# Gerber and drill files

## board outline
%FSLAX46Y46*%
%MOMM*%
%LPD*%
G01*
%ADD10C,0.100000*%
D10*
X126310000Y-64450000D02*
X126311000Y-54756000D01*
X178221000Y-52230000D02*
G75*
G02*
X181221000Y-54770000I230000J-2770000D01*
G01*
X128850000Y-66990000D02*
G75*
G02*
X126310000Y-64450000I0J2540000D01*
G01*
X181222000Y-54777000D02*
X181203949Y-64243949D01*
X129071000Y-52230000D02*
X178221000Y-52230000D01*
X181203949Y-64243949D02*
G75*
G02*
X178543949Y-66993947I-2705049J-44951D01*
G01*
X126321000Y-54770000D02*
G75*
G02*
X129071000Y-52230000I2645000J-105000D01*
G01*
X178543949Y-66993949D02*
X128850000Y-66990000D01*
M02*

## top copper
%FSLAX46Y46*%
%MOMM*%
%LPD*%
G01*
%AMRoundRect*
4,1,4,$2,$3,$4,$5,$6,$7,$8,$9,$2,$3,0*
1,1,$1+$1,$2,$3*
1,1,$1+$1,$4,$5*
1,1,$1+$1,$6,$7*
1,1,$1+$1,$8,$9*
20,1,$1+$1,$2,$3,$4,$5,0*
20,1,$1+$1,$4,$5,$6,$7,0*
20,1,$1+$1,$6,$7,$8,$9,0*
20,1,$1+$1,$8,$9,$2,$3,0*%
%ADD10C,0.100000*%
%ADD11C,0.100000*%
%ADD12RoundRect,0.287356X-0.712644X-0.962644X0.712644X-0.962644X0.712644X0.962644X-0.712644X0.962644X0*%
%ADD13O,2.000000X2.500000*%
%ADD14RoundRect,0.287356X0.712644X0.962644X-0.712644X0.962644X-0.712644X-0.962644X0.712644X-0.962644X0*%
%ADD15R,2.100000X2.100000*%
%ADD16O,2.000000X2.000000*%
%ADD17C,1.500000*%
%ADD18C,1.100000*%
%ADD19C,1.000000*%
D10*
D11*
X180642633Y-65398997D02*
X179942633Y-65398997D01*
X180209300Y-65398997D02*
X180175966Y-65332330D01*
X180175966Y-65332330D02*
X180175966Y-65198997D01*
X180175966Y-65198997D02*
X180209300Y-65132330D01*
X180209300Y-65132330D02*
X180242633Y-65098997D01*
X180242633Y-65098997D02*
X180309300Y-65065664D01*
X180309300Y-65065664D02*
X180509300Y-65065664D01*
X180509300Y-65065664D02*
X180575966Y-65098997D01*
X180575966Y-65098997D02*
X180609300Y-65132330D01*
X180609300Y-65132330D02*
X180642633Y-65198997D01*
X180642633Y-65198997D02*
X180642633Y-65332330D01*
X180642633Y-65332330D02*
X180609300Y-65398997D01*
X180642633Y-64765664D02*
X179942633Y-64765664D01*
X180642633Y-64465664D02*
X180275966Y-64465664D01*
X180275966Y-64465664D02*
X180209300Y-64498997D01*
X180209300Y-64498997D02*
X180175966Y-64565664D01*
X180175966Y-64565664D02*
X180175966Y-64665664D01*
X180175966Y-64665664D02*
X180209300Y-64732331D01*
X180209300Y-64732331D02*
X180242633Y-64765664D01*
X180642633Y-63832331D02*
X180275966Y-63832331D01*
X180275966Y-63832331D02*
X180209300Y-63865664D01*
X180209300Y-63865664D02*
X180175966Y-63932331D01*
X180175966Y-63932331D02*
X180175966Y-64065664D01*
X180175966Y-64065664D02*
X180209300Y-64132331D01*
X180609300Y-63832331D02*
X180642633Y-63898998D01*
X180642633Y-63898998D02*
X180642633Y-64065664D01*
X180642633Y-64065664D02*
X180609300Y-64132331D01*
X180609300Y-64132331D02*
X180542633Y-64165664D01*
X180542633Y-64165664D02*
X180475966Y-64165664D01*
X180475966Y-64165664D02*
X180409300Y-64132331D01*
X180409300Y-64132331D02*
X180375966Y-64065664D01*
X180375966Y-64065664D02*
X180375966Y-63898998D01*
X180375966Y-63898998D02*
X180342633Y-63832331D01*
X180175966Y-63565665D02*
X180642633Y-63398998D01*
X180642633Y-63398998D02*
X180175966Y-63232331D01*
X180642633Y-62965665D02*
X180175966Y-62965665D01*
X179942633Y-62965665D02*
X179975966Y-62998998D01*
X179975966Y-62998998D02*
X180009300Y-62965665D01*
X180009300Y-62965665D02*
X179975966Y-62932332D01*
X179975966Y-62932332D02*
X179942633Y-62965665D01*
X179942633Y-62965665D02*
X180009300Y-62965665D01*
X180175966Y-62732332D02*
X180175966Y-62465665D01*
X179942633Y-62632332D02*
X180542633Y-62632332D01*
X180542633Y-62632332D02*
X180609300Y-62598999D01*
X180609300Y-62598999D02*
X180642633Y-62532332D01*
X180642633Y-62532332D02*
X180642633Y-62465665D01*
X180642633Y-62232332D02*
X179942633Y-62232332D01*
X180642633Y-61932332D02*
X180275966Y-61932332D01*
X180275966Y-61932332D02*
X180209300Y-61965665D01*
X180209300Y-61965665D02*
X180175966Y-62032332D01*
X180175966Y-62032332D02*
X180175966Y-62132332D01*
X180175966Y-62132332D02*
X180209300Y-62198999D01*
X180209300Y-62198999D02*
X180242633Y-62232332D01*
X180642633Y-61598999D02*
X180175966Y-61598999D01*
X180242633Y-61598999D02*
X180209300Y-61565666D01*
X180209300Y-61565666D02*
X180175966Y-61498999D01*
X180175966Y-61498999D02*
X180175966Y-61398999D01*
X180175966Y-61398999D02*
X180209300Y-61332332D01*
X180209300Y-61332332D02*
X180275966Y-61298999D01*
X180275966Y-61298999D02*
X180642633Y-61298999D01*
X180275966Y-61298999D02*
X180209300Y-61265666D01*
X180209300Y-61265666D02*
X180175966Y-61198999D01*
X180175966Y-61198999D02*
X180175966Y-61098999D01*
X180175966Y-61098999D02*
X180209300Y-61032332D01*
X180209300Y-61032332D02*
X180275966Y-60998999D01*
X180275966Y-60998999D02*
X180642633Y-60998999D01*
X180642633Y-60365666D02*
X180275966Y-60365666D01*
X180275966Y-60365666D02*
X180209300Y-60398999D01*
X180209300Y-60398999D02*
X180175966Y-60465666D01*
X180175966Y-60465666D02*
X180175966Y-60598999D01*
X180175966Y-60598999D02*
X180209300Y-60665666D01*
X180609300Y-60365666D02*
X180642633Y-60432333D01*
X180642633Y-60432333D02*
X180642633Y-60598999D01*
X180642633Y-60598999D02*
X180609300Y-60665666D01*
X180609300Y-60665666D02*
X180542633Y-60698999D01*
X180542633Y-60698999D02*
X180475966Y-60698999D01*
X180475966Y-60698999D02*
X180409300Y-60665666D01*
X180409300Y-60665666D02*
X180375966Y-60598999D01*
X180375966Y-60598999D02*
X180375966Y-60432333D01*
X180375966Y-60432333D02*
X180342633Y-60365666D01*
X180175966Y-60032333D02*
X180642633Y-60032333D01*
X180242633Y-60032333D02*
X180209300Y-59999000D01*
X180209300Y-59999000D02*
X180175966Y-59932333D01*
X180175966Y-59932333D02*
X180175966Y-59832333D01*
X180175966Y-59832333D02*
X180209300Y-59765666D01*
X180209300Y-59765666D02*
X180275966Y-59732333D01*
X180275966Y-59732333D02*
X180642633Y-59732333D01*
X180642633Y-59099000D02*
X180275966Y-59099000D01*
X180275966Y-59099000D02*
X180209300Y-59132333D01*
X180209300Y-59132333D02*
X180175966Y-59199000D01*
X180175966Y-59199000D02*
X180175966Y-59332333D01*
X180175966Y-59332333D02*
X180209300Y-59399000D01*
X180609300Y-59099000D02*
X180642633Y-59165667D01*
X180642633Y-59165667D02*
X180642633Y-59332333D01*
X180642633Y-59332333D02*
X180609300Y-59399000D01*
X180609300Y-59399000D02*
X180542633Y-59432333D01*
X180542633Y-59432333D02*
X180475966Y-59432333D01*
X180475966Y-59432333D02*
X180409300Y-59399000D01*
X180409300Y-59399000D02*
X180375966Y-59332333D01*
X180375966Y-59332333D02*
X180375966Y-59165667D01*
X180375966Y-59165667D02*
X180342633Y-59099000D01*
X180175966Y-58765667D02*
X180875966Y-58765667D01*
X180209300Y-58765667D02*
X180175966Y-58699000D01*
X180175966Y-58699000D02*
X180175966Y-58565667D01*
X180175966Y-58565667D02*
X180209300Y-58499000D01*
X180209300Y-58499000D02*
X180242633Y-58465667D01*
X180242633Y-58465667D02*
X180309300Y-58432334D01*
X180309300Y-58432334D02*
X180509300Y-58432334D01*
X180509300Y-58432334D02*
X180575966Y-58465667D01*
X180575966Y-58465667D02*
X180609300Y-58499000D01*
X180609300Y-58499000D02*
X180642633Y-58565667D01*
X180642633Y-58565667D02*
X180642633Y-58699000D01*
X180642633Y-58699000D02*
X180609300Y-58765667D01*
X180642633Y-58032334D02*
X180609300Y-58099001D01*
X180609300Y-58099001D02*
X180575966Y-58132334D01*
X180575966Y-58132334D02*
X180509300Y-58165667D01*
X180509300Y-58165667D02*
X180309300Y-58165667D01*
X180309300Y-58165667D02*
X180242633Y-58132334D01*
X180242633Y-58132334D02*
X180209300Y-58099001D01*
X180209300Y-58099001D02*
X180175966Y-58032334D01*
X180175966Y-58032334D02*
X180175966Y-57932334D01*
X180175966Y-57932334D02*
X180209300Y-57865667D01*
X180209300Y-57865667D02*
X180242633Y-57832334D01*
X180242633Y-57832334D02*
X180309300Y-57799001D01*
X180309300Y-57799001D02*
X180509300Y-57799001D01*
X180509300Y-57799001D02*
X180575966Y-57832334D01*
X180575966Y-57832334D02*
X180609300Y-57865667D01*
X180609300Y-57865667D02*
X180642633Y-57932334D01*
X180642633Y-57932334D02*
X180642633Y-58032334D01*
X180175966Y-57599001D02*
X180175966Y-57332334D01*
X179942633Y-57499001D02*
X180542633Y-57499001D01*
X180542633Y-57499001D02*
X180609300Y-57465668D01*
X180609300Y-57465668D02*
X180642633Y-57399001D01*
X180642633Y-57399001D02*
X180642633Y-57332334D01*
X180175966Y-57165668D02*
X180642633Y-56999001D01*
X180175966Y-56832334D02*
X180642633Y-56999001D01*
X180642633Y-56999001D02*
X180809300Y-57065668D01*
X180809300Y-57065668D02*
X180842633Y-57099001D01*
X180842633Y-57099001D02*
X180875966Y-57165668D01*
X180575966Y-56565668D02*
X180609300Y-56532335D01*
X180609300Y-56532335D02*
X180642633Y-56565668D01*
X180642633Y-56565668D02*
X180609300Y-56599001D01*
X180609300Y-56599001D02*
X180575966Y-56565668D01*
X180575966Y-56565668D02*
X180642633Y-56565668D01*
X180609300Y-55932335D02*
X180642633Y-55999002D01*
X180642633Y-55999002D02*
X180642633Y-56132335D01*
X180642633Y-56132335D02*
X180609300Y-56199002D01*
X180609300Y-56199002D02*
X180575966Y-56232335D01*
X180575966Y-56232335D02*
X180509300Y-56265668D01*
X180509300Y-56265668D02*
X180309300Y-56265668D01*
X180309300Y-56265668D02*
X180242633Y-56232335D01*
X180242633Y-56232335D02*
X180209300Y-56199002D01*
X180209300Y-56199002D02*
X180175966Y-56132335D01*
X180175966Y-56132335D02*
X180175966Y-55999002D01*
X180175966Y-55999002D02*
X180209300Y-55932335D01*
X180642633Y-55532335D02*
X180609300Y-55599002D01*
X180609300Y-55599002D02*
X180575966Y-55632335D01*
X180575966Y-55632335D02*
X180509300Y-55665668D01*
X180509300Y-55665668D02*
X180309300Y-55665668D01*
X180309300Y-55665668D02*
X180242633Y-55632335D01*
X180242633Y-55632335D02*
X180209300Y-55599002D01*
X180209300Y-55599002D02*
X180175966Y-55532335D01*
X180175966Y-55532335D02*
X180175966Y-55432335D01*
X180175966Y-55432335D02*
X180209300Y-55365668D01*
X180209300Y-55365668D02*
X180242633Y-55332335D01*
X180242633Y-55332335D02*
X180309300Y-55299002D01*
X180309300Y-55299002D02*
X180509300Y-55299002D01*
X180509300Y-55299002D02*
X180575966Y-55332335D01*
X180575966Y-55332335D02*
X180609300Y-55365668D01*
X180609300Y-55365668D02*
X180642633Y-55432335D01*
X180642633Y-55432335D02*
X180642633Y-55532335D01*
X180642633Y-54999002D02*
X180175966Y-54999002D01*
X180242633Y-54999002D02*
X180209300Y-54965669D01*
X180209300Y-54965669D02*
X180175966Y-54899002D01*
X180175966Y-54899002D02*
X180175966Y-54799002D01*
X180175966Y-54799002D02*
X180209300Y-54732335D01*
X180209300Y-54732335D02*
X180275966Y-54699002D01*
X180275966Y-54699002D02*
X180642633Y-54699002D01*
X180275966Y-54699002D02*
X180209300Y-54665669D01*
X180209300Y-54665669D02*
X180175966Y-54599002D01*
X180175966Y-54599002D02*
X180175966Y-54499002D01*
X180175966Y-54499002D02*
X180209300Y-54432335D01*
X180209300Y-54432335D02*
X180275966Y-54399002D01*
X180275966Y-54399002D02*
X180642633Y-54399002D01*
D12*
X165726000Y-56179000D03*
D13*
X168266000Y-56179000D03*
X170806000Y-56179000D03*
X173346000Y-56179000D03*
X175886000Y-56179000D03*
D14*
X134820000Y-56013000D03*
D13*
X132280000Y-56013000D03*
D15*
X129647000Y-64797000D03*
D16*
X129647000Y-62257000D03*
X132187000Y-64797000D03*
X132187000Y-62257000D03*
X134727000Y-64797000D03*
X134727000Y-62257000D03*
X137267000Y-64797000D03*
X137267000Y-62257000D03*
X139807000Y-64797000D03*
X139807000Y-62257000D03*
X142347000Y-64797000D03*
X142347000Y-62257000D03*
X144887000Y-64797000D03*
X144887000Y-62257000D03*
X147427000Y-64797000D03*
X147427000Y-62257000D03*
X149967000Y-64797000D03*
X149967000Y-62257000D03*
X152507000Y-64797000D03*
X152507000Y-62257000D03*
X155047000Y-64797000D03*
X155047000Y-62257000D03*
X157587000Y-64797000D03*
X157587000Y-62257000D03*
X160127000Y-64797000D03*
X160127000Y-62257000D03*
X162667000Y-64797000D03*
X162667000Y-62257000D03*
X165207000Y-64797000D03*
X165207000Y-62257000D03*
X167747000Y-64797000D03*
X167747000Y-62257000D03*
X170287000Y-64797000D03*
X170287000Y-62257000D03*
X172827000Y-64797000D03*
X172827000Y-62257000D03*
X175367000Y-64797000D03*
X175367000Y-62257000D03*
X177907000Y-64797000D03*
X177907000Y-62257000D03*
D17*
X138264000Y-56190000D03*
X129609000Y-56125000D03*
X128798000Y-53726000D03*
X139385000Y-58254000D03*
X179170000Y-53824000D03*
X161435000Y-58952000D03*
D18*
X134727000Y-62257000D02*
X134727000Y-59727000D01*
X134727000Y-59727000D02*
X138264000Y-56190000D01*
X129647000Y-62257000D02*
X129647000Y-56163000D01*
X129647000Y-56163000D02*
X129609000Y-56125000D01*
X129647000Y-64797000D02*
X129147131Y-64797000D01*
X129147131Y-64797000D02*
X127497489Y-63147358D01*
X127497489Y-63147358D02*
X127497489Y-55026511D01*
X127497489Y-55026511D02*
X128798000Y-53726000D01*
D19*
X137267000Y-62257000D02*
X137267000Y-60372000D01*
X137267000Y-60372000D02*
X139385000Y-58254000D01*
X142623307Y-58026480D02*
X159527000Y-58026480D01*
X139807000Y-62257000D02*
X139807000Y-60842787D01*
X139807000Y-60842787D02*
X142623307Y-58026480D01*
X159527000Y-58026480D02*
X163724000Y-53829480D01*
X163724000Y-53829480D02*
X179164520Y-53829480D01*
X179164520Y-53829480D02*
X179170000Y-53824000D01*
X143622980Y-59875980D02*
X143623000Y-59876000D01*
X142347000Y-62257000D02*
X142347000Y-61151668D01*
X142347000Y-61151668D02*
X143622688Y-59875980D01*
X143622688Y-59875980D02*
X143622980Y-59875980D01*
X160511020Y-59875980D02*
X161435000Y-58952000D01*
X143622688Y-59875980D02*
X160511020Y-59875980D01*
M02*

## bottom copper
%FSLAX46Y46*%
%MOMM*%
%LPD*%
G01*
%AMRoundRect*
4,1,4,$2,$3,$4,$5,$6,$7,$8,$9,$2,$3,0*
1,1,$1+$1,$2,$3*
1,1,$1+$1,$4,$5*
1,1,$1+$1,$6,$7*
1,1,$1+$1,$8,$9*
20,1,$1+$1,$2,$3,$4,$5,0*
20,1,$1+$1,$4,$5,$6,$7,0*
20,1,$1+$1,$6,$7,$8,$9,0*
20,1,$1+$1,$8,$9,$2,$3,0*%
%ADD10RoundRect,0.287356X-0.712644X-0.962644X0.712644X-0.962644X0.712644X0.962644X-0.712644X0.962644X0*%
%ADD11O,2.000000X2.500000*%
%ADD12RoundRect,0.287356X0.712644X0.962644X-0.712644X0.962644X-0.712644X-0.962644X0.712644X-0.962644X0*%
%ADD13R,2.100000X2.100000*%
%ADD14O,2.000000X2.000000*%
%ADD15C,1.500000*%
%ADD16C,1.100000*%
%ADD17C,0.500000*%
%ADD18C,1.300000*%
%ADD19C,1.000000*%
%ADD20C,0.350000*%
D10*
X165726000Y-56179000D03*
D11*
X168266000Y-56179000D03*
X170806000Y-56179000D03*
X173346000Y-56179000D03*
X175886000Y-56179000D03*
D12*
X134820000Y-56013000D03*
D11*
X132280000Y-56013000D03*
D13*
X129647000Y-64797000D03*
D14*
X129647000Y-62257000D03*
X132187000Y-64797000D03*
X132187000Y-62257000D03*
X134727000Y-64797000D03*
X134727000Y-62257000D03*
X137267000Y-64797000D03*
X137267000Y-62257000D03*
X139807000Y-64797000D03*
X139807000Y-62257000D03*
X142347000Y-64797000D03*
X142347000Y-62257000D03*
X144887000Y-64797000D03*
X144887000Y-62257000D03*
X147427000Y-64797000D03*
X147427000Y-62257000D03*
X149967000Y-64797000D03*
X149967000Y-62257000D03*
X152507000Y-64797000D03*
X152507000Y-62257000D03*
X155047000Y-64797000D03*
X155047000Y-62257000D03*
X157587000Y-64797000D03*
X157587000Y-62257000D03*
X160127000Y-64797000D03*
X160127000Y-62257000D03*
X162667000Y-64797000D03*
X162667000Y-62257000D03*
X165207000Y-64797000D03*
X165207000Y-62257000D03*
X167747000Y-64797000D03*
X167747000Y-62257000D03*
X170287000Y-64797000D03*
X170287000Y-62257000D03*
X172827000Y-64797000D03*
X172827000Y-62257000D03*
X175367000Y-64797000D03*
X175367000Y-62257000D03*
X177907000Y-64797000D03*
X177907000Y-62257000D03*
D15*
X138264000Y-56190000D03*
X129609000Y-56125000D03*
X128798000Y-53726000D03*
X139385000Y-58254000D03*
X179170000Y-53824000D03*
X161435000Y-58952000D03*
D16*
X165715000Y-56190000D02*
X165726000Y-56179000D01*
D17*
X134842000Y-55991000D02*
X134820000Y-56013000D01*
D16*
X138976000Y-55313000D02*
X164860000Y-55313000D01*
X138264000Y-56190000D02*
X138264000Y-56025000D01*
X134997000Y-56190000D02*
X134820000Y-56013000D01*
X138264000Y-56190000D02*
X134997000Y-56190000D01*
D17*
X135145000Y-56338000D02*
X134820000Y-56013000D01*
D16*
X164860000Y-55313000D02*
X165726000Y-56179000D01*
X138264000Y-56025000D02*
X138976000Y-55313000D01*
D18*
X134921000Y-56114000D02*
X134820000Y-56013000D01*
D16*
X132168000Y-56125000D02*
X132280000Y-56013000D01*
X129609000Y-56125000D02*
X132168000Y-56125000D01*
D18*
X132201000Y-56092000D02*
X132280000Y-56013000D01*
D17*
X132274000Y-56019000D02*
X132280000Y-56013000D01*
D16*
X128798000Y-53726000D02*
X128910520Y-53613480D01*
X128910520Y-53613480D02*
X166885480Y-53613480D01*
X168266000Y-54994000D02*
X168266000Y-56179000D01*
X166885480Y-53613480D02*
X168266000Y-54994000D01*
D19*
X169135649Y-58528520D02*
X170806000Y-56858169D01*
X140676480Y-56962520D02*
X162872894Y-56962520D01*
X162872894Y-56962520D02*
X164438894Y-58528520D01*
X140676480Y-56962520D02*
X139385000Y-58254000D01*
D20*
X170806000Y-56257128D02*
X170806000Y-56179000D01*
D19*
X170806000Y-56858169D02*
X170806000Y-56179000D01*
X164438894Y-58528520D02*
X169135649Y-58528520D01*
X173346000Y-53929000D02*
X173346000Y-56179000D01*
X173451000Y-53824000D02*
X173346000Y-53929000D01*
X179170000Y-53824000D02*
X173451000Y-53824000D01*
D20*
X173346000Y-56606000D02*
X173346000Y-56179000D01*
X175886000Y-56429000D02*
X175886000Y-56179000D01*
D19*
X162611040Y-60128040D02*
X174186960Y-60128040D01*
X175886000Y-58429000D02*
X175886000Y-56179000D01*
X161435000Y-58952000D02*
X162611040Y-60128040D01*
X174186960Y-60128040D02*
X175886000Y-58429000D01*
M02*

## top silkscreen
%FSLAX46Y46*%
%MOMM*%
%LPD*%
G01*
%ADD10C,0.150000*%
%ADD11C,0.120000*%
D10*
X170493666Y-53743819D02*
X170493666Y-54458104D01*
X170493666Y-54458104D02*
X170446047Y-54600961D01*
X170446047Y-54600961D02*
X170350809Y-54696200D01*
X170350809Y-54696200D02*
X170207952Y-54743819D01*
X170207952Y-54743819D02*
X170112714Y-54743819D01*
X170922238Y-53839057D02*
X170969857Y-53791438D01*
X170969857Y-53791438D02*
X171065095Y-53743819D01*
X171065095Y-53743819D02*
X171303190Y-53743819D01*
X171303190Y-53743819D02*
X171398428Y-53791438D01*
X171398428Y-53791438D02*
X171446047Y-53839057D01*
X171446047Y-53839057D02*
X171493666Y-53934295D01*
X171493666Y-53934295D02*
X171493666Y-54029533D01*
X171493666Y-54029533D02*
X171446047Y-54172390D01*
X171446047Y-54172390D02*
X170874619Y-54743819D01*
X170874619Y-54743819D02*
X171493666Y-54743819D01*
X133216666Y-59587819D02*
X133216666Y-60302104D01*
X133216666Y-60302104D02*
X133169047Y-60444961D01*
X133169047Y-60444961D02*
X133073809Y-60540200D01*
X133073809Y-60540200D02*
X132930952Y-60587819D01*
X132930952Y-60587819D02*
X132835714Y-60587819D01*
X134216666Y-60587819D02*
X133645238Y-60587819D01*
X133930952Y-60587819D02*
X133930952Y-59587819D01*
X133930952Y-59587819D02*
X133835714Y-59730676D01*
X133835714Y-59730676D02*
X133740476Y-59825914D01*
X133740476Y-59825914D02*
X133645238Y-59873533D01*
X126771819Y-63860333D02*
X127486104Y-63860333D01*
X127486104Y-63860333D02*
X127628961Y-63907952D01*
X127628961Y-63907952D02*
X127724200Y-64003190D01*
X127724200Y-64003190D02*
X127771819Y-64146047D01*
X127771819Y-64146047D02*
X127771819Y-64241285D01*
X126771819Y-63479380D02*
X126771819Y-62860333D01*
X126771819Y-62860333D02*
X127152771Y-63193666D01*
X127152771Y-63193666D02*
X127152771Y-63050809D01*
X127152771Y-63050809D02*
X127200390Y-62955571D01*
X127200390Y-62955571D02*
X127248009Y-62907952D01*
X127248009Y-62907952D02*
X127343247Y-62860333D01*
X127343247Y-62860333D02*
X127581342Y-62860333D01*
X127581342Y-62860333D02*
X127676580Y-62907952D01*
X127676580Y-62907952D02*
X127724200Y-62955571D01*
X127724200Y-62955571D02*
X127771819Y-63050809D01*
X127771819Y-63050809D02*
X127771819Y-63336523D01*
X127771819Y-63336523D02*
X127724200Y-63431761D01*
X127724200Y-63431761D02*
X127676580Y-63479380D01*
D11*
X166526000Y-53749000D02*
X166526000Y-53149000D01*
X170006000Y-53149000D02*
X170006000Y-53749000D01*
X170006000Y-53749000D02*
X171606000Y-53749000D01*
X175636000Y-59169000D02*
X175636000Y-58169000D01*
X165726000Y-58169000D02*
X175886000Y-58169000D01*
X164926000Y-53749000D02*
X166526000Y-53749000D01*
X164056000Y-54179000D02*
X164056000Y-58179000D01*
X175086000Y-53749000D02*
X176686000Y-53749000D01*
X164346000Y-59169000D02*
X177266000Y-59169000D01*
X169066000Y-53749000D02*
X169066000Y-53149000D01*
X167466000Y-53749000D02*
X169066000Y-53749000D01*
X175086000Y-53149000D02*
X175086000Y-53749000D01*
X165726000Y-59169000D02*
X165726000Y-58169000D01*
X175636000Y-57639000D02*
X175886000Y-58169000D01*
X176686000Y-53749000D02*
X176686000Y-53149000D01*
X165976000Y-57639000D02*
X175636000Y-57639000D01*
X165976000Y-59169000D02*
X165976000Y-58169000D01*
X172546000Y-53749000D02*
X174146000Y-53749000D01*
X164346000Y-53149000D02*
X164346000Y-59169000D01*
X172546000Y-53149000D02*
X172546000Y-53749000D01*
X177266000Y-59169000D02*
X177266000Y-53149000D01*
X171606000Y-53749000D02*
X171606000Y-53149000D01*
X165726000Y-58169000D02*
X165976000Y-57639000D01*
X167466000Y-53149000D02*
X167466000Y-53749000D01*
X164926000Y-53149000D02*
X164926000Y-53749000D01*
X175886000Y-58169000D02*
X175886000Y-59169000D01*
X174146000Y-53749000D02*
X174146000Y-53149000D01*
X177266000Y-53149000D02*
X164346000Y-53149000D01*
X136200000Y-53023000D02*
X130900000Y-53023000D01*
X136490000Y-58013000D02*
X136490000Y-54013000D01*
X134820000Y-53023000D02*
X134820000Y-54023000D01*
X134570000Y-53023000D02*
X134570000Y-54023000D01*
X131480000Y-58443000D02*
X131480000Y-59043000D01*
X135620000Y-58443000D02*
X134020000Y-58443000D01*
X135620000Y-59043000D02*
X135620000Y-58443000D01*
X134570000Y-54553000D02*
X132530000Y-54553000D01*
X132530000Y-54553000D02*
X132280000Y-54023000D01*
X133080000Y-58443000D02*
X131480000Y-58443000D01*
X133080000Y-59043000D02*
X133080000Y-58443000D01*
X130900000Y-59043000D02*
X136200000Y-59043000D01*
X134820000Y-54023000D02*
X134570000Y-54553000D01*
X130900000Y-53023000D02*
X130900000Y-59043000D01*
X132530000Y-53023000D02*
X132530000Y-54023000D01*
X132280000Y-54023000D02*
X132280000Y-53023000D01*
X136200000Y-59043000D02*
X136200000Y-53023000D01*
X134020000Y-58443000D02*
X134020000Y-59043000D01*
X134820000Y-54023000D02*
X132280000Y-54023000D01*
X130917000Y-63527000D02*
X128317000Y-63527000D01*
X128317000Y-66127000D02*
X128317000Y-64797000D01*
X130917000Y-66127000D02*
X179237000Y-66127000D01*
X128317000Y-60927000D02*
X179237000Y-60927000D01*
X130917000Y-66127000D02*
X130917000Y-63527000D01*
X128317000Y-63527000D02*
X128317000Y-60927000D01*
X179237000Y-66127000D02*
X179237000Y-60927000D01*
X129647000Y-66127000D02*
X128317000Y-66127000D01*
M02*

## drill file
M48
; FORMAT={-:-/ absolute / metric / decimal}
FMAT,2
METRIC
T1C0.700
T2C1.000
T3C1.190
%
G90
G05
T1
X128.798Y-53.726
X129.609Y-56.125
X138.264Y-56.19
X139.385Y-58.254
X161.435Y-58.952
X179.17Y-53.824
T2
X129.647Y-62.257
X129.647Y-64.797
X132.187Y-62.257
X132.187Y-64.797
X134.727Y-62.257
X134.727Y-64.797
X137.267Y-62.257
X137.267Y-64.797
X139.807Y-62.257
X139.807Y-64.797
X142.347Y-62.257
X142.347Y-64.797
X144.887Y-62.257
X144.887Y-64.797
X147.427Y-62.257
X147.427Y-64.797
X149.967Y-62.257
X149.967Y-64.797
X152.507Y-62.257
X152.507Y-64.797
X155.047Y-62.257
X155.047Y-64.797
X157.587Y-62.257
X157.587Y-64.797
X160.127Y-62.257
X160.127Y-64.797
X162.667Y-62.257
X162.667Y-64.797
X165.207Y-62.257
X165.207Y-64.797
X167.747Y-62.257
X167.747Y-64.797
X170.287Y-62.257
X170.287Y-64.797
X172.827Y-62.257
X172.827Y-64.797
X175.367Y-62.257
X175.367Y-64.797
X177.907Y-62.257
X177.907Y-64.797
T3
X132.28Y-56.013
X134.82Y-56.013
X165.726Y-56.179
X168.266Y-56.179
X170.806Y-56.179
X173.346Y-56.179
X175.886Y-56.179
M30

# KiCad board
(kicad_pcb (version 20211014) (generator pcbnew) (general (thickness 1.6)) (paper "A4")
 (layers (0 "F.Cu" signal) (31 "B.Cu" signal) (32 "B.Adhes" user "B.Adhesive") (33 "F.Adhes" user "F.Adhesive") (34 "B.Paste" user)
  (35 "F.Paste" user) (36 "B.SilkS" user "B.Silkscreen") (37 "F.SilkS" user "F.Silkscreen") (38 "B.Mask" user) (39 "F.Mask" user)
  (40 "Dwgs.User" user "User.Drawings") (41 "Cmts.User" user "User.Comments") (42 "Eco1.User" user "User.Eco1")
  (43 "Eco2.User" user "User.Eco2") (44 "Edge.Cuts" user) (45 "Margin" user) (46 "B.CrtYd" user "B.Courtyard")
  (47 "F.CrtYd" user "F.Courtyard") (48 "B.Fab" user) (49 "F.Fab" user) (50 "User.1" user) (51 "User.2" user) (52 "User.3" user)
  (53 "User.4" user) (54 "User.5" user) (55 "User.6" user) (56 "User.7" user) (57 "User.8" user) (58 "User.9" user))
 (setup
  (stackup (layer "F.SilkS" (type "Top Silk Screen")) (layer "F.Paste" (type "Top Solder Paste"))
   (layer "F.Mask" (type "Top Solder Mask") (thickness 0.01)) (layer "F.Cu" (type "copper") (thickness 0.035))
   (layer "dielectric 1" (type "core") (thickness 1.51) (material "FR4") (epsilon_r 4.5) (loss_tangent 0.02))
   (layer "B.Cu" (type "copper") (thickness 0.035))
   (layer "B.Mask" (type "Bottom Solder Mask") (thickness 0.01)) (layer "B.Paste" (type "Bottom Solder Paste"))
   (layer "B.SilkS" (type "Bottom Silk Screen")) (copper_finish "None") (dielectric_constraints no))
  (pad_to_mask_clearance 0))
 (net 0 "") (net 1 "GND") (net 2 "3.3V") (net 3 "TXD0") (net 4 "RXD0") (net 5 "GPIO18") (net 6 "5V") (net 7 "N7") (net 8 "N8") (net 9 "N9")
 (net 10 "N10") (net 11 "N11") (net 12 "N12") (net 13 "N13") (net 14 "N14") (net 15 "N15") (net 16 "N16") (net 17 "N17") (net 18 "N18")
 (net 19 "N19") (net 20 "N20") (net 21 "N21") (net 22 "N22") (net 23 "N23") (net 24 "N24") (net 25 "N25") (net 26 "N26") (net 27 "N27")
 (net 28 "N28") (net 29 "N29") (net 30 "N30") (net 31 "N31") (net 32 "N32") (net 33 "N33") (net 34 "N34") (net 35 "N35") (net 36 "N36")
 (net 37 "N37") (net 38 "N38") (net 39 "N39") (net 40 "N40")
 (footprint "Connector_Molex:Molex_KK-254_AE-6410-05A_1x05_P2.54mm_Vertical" (layer "F.Cu") (at 165.726 56.179)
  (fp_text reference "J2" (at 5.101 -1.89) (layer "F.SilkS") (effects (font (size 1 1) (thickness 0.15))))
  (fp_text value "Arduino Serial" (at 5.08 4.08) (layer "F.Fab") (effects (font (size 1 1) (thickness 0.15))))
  (fp_line (start 0.8 -2.43) (end 0.8 -3.03) (layer "F.SilkS") (width 0.12))
  (fp_line (start 4.28 -3.03) (end 4.28 -2.43) (layer "F.SilkS") (width 0.12))
  (fp_line (start 4.28 -2.43) (end 5.88 -2.43) (layer "F.SilkS") (width 0.12))
  (fp_line (start 9.91 2.99) (end 9.91 1.99) (layer "F.SilkS") (width 0.12))
  (fp_line (start 0 1.99) (end 10.16 1.99) (layer "F.SilkS") (width 0.12))
  (fp_line (start -0.8 -2.43) (end 0.8 -2.43) (layer "F.SilkS") (width 0.12))
  (fp_line (start -1.67 -2) (end -1.67 2) (layer "F.SilkS") (width 0.12))
  (fp_line (start 9.36 -2.43) (end 10.96 -2.43) (layer "F.SilkS") (width 0.12))
  (fp_line (start -1.38 2.99) (end 11.54 2.99) (layer "F.SilkS") (width 0.12))
  (fp_line (start 3.34 -2.43) (end 3.34 -3.03) (layer "F.SilkS") (width 0.12))
  (fp_line (start 1.74 -2.43) (end 3.34 -2.43) (layer "F.SilkS") (width 0.12))
  (fp_line (start 9.36 -3.03) (end 9.36 -2.43) (layer "F.SilkS") (width 0.12))
  (fp_line (start 0 2.99) (end 0 1.99) (layer "F.SilkS") (width 0.12))
  (fp_line (start 9.91 1.46) (end 10.16 1.99) (layer "F.SilkS") (width 0.12))
  (fp_line (start 10.96 -2.43) (end 10.96 -3.03) (layer "F.SilkS") (width 0.12))
  (fp_line (start 0.25 1.46) (end 9.91 1.46) (layer "F.SilkS") (width 0.12))
  (fp_line (start 0.25 2.99) (end 0.25 1.99) (layer "F.SilkS") (width 0.12))
  (fp_line (start 6.82 -2.43) (end 8.42 -2.43) (layer "F.SilkS") (width 0.12))
  (fp_line (start -1.38 -3.03) (end -1.38 2.99) (layer "F.SilkS") (width 0.12))
  (fp_line (start 6.82 -3.03) (end 6.82 -2.43) (layer "F.SilkS") (width 0.12))
  (fp_line (start 11.54 2.99) (end 11.54 -3.03) (layer "F.SilkS") (width 0.12))
  (fp_line (start 5.88 -2.43) (end 5.88 -3.03) (layer "F.SilkS") (width 0.12))
  (fp_line (start 0 1.99) (end 0.25 1.46) (layer "F.SilkS") (width 0.12))
  (fp_line (start 1.74 -3.03) (end 1.74 -2.43) (layer "F.SilkS") (width 0.12))
  (fp_line (start -0.8 -3.03) (end -0.8 -2.43) (layer "F.SilkS") (width 0.12))
  (fp_line (start 10.16 1.99) (end 10.16 2.99) (layer "F.SilkS") (width 0.12))
  (fp_line (start 8.42 -2.43) (end 8.42 -3.03) (layer "F.SilkS") (width 0.12))
  (fp_line (start 11.54 -3.03) (end -1.38 -3.03) (layer "F.SilkS") (width 0.12))
  (pad "1" thru_hole roundrect (at 0 0) (size 2 2.5) (drill 1.19) (layers *.Cu *.Mask) (roundrect_rratio 0.143678) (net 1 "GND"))
  (pad "2" thru_hole oval (at 2.54 0) (size 2 2.5) (drill 1.19) (layers *.Cu *.Mask) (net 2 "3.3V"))
  (pad "3" thru_hole oval (at 5.08 0) (size 2 2.5) (drill 1.19) (layers *.Cu *.Mask) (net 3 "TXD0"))
  (pad "4" thru_hole oval (at 7.62 0) (size 2 2.5) (drill 1.19) (layers *.Cu *.Mask) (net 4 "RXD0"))
  (pad "5" thru_hole oval (at 10.16 0) (size 2 2.5) (drill 1.19) (layers *.Cu *.Mask) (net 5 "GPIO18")))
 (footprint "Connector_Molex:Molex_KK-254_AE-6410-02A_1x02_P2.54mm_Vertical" (layer "F.Cu") (at 134.82 56.013 180)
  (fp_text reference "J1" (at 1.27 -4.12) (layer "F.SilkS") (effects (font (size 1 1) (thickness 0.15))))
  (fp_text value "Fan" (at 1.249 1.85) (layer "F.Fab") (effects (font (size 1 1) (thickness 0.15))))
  (fp_line (start -1.38 2.99) (end 3.92 2.99) (layer "F.SilkS") (width 0.12))
  (fp_line (start -1.67 -2) (end -1.67 2) (layer "F.SilkS") (width 0.12))
  (fp_line (start 0 2.99) (end 0 1.99) (layer "F.SilkS") (width 0.12))
  (fp_line (start 0.25 2.99) (end 0.25 1.99) (layer "F.SilkS") (width 0.12))
  (fp_line (start 3.34 -2.43) (end 3.34 -3.03) (layer "F.SilkS") (width 0.12))
  (fp_line (start -0.8 -2.43) (end 0.8 -2.43) (layer "F.SilkS") (width 0.12))
  (fp_line (start -0.8 -3.03) (end -0.8 -2.43) (layer "F.SilkS") (width 0.12))
  (fp_line (start 0.25 1.46) (end 2.29 1.46) (layer "F.SilkS") (width 0.12))
  (fp_line (start 2.29 1.46) (end 2.54 1.99) (layer "F.SilkS") (width 0.12))
  (fp_line (start 1.74 -2.43) (end 3.34 -2.43) (layer "F.SilkS") (width 0.12))
  (fp_line (start 1.74 -3.03) (end 1.74 -2.43) (layer "F.SilkS") (width 0.12))
  (fp_line (start 3.92 -3.03) (end -1.38 -3.03) (layer "F.SilkS") (width 0.12))
  (fp_line (start 0 1.99) (end 0.25 1.46) (layer "F.SilkS") (width 0.12))
  (fp_line (start 3.92 2.99) (end 3.92 -3.03) (layer "F.SilkS") (width 0.12))
  (fp_line (start 2.29 2.99) (end 2.29 1.99) (layer "F.SilkS") (width 0.12))
  (fp_line (start 2.54 1.99) (end 2.54 2.99) (layer "F.SilkS") (width 0.12))
  (fp_line (start -1.38 -3.03) (end -1.38 2.99) (layer "F.SilkS") (width 0.12))
  (fp_line (start 0.8 -2.43) (end 0.8 -3.03) (layer "F.SilkS") (width 0.12))
  (fp_line (start 0 1.99) (end 2.54 1.99) (layer "F.SilkS") (width 0.12))
  (pad "1" thru_hole roundrect (at 0 0 180) (size 2 2.5) (drill 1.19) (layers *.Cu *.Mask) (roundrect_rratio 0.143678) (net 1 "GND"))
  (pad "2" thru_hole oval (at 2.54 0 180) (size 2 2.5) (drill 1.19) (layers *.Cu *.Mask) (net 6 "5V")))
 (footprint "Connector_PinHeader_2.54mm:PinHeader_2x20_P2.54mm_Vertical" (layer "F.Cu") (at 129.647 64.797 90)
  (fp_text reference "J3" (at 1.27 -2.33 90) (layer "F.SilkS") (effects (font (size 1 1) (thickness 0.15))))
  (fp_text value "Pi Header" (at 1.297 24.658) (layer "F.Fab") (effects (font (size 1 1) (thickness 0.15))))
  (fp_line (start 1.27 1.27) (end 1.27 -1.33) (layer "F.SilkS") (width 0.12))
  (fp_line (start -1.33 -1.33) (end 0 -1.33) (layer "F.SilkS") (width 0.12))
  (fp_line (start -1.33 1.27) (end -1.33 49.59) (layer "F.SilkS") (width 0.12))
  (fp_line (start 3.87 -1.33) (end 3.87 49.59) (layer "F.SilkS") (width 0.12))
  (fp_line (start -1.33 1.27) (end 1.27 1.27) (layer "F.SilkS") (width 0.12))
  (fp_line (start 1.27 -1.33) (end 3.87 -1.33) (layer "F.SilkS") (width 0.12))
  (fp_line (start -1.33 49.59) (end 3.87 49.59) (layer "F.SilkS") (width 0.12))
  (fp_line (start -1.33 0) (end -1.33 -1.33) (layer "F.SilkS") (width 0.12))
  (pad "1" thru_hole rect (at 0 0 90) (size 2.1 2.1) (drill 1) (layers *.Cu *.Mask) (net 2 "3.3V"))
  (pad "2" thru_hole oval (at 2.54 0 90) (size 2 2) (drill 1) (layers *.Cu *.Mask) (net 6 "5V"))
  (pad "3" thru_hole oval (at 0 2.54 90) (size 2 2) (drill 1) (layers *.Cu *.Mask) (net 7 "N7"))
  (pad "4" thru_hole oval (at 2.54 2.54 90) (size 2 2) (drill 1) (layers *.Cu *.Mask) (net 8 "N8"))
  (pad "5" thru_hole oval (at 0 5.08 90) (size 2 2) (drill 1) (layers *.Cu *.Mask) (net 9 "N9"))
  (pad "6" thru_hole oval (at 2.54 5.08 90) (size 2 2) (drill 1) (layers *.Cu *.Mask) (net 1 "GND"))
  (pad "7" thru_hole oval (at 0 7.62 90) (size 2 2) (drill 1) (layers *.Cu *.Mask) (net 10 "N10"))
  (pad "8" thru_hole oval (at 2.54 7.62 90) (size 2 2) (drill 1) (layers *.Cu *.Mask) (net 3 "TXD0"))
  (pad "9" thru_hole oval (at 0 10.16 90) (size 2 2) (drill 1) (layers *.Cu *.Mask) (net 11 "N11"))
  (pad "10" thru_hole oval (at 2.54 10.16 90) (size 2 2) (drill 1) (layers *.Cu *.Mask) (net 4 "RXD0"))
  (pad "11" thru_hole oval (at 0 12.7 90) (size 2 2) (drill 1) (layers *.Cu *.Mask) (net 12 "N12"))
  (pad "12" thru_hole oval (at 2.54 12.7 90) (size 2 2) (drill 1) (layers *.Cu *.Mask) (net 5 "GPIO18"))
  (pad "13" thru_hole oval (at 0 15.24 90) (size 2 2) (drill 1) (layers *.Cu *.Mask) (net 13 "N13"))
  (pad "14" thru_hole oval (at 2.54 15.24 90) (size 2 2) (drill 1) (layers *.Cu *.Mask) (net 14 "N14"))
  (pad "15" thru_hole oval (at 0 17.78 90) (size 2 2) (drill 1) (layers *.Cu *.Mask) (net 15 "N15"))
  (pad "16" thru_hole oval (at 2.54 17.78 90) (size 2 2) (drill 1) (layers *.Cu *.Mask) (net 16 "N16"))
  (pad "17" thru_hole oval (at 0 20.32 90) (size 2 2) (drill 1) (layers *.Cu *.Mask) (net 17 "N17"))
  (pad "18" thru_hole oval (at 2.54 20.32 90) (size 2 2) (drill 1) (layers *.Cu *.Mask) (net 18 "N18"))
  (pad "19" thru_hole oval (at 0 22.86 90) (size 2 2) (drill 1) (layers *.Cu *.Mask) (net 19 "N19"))
  (pad "20" thru_hole oval (at 2.54 22.86 90) (size 2 2) (drill 1) (layers *.Cu *.Mask) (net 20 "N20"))
  (pad "21" thru_hole oval (at 0 25.4 90) (size 2 2) (drill 1) (layers *.Cu *.Mask) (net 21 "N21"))
  (pad "22" thru_hole oval (at 2.54 25.4 90) (size 2 2) (drill 1) (layers *.Cu *.Mask) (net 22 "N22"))
  (pad "23" thru_hole oval (at 0 27.94 90) (size 2 2) (drill 1) (layers *.Cu *.Mask) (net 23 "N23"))
  (pad "24" thru_hole oval (at 2.54 27.94 90) (size 2 2) (drill 1) (layers *.Cu *.Mask) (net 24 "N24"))
  (pad "25" thru_hole oval (at 0 30.48 90) (size 2 2) (drill 1) (layers *.Cu *.Mask) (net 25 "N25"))
  (pad "26" thru_hole oval (at 2.54 30.48 90) (size 2 2) (drill 1) (layers *.Cu *.Mask) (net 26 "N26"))
  (pad "27" thru_hole oval (at 0 33.02 90) (size 2 2) (drill 1) (layers *.Cu *.Mask) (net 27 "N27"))
  (pad "28" thru_hole oval (at 2.54 33.02 90) (size 2 2) (drill 1) (layers *.Cu *.Mask) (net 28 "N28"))
  (pad "29" thru_hole oval (at 0 35.56 90) (size 2 2) (drill 1) (layers *.Cu *.Mask) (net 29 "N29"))
  (pad "30" thru_hole oval (at 2.54 35.56 90) (size 2 2) (drill 1) (layers *.Cu *.Mask) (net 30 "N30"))
  (pad "31" thru_hole oval (at 0 38.1 90) (size 2 2) (drill 1) (layers *.Cu *.Mask) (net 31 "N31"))
  (pad "32" thru_hole oval (at 2.54 38.1 90) (size 2 2) (drill 1) (layers *.Cu *.Mask) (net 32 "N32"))
  (pad "33" thru_hole oval (at 0 40.64 90) (size 2 2) (drill 1) (layers *.Cu *.Mask) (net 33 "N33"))
  (pad "34" thru_hole oval (at 2.54 40.64 90) (size 2 2) (drill 1) (layers *.Cu *.Mask) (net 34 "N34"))
  (pad "35" thru_hole oval (at 0 43.18 90) (size 2 2) (drill 1) (layers *.Cu *.Mask) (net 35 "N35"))
  (pad "36" thru_hole oval (at 2.54 43.18 90) (size 2 2) (drill 1) (layers *.Cu *.Mask) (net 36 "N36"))
  (pad "37" thru_hole oval (at 0 45.72 90) (size 2 2) (drill 1) (layers *.Cu *.Mask) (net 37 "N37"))
  (pad "38" thru_hole oval (at 2.54 45.72 90) (size 2 2) (drill 1) (layers *.Cu *.Mask) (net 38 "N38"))
  (pad "39" thru_hole oval (at 0 48.26 90) (size 2 2) (drill 1) (layers *.Cu *.Mask) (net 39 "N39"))
  (pad "40" thru_hole oval (at 2.54 48.26 90) (size 2 2) (drill 1) (layers *.Cu *.Mask) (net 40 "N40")))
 (gr_line (start 126.31 64.45) (end 126.311 54.756) (layer "Edge.Cuts") (width 0.1))
 (gr_arc (start 178.221 52.23) (mid 180.247051 52.87868) (end 181.221 54.77) (layer "Edge.Cuts") (width 0.1))
 (gr_arc (start 128.85 66.99) (mid 127.053949 66.246051) (end 126.31 64.45) (layer "Edge.Cuts") (width 0.1))
 (gr_line (start 181.222 54.777) (end 181.203949 64.243949) (layer "Edge.Cuts") (width 0.1))
 (gr_line (start 129.071 52.23) (end 178.221 52.23) (layer "Edge.Cuts") (width 0.1))
 (gr_arc (start 181.203949 64.243949) (mid 180.443493 66.169853) (end 178.543949 66.993949) (layer "Edge.Cuts") (width 0.1))
 (gr_arc (start 126.321 54.77) (mid 127.169949 52.930456) (end 129.071 52.23) (layer "Edge.Cuts") (width 0.1))
 (gr_line (start 178.543949 66.993949) (end 128.85 66.99) (layer "Edge.Cuts") (width 0.1))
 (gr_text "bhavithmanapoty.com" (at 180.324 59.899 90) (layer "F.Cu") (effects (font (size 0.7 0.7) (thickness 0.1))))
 (segment (start 134.727 62.257) (end 134.727 59.727) (width 1.1) (layer "F.Cu") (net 1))
 (segment (start 134.727 59.727) (end 138.264 56.19) (width 1.1) (layer "F.Cu") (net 1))
 (via (at 138.264 56.19) (size 1.5) (drill 0.7) (layers "F.Cu" "B.Cu") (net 1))
 (segment (start 165.715 56.19) (end 165.726 56.179) (width 1.1) (layer "B.Cu") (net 1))
 (segment (start 134.842 55.991) (end 134.82 56.013) (width 0.5) (layer "B.Cu") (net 1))
 (segment (start 138.976 55.313) (end 164.86 55.313) (width 1.1) (layer "B.Cu") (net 1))
 (segment (start 138.264 56.19) (end 138.264 56.025) (width 1.1) (layer "B.Cu") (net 1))
 (segment (start 134.997 56.19) (end 134.82 56.013) (width 1.1) (layer "B.Cu") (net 1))
 (segment (start 138.264 56.19) (end 134.997 56.19) (width 1.1) (layer "B.Cu") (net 1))
 (segment (start 135.145 56.338) (end 134.82 56.013) (width 0.5) (layer "B.Cu") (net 1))
 (segment (start 164.86 55.313) (end 165.726 56.179) (width 1.1) (layer "B.Cu") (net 1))
 (segment (start 138.264 56.025) (end 138.976 55.313) (width 1.1) (layer "B.Cu") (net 1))
 (segment (start 134.921 56.114) (end 134.82 56.013) (width 1.3) (layer "B.Cu") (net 1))
 (segment (start 129.647 62.257) (end 129.647 56.163) (width 1.1) (layer "F.Cu") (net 6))
 (segment (start 129.647 56.163) (end 129.609 56.125) (width 1.1) (layer "F.Cu") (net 6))
 (via (at 129.609 56.125) (size 1.5) (drill 0.7) (layers "F.Cu" "B.Cu") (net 6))
 (segment (start 132.168 56.125) (end 132.28 56.013) (width 1.1) (layer "B.Cu") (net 6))
 (segment (start 129.609 56.125) (end 132.168 56.125) (width 1.1) (layer "B.Cu") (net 6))
 (segment (start 132.201 56.092) (end 132.28 56.013) (width 1.3) (layer "B.Cu") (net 6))
 (segment (start 132.274 56.019) (end 132.28 56.013) (width 0.5) (layer "B.Cu") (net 6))
 (segment (start 129.647 64.797) (end 129.147131 64.797) (width 1.1) (layer "F.Cu") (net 2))
 (segment (start 129.147131 64.797) (end 127.497489 63.147358) (width 1.1) (layer "F.Cu") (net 2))
 (segment (start 127.497489 63.147358) (end 127.497489 55.026511) (width 1.1) (layer "F.Cu") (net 2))
 (segment (start 127.497489 55.026511) (end 128.798 53.726) (width 1.1) (layer "F.Cu") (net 2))
 (via (at 128.798 53.726) (size 1.5) (drill 0.7) (layers "F.Cu" "B.Cu") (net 2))
 (segment (start 128.798 53.726) (end 128.91052 53.61348) (width 1.1) (layer "B.Cu") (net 2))
 (segment (start 128.91052 53.61348) (end 166.88548 53.61348) (width 1.1) (layer "B.Cu") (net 2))
 (segment (start 168.266 54.994) (end 168.266 56.179) (width 1.1) (layer "B.Cu") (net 2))
 (segment (start 166.88548 53.61348) (end 168.266 54.994) (width 1.1) (layer "B.Cu") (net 2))
 (segment (start 137.267 62.257) (end 137.267 60.372) (width 1) (layer "F.Cu") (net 3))
 (segment (start 137.267 60.372) (end 139.385 58.254) (width 1) (layer "F.Cu") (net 3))
 (via (at 139.385 58.254) (size 1.5) (drill 0.7) (layers "F.Cu" "B.Cu") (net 3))
 (segment (start 169.135649 58.52852) (end 170.806 56.858169) (width 1) (layer "B.Cu") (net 3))
 (segment (start 140.67648 56.96252) (end 162.872894 56.96252) (width 1) (layer "B.Cu") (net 3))
 (segment (start 162.872894 56.96252) (end 164.438894 58.52852) (width 1) (layer "B.Cu") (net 3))
 (segment (start 140.67648 56.96252) (end 139.385 58.254) (width 1) (layer "B.Cu") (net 3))
 (segment (start 170.806 56.257128) (end 170.806 56.179) (width 0.35) (layer "B.Cu") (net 3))
 (segment (start 170.806 56.858169) (end 170.806 56.179) (width 1) (layer "B.Cu") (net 3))
 (segment (start 164.438894 58.52852) (end 169.135649 58.52852) (width 1) (layer "B.Cu") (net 3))
 (segment (start 142.623307 58.02648) (end 159.527 58.02648) (width 1) (layer "F.Cu") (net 4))
 (segment (start 139.807 62.257) (end 139.807 60.842787) (width 1) (layer "F.Cu") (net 4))
 (segment (start 139.807 60.842787) (end 142.623307 58.02648) (width 1) (layer "F.Cu") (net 4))
 (segment (start 159.527 58.02648) (end 163.724 53.82948) (width 1) (layer "F.Cu") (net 4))
 (segment (start 163.724 53.82948) (end 179.16452 53.82948) (width 1) (layer "F.Cu") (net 4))
 (segment (start 179.16452 53.82948) (end 179.17 53.824) (width 1) (layer "F.Cu") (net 4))
 (via (at 179.17 53.824) (size 1.5) (drill 0.7) (layers "F.Cu" "B.Cu") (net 4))
 (segment (start 173.346 53.929) (end 173.346 56.179) (width 1) (layer "B.Cu") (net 4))
 (segment (start 173.451 53.824) (end 173.346 53.929) (width 1) (layer "B.Cu") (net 4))
 (segment (start 179.17 53.824) (end 173.451 53.824) (width 1) (layer "B.Cu") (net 4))
 (segment (start 173.346 56.606) (end 173.346 56.179) (width 0.35) (layer "B.Cu") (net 4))
 (segment (start 143.62298 59.87598) (end 143.623 59.876) (width 1) (layer "F.Cu") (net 5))
 (segment (start 142.347 62.257) (end 142.347 61.151668) (width 1) (layer "F.Cu") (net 5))
 (segment (start 142.347 61.151668) (end 143.622688 59.87598) (width 1) (layer "F.Cu") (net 5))
 (segment (start 143.622688 59.87598) (end 143.62298 59.87598) (width 1) (layer "F.Cu") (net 5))
 (segment (start 160.51102 59.87598) (end 161.435 58.952) (width 1) (layer "F.Cu") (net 5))
 (segment (start 143.622688 59.87598) (end 160.51102 59.87598) (width 1) (layer "F.Cu") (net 5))
 (via (at 161.435 58.952) (size 1.5) (drill 0.7) (layers "F.Cu" "B.Cu") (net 5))
 (segment (start 175.886 56.429) (end 175.886 56.179) (width 0.35) (layer "B.Cu") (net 5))
 (segment (start 162.61104 60.12804) (end 174.18696 60.12804) (width 1) (layer "B.Cu") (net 5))
 (segment (start 175.886 58.429) (end 175.886 56.179) (width 1) (layer "B.Cu") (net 5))
 (segment (start 161.435 58.952) (end 162.61104 60.12804) (width 1) (layer "B.Cu") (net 5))
 (segment (start 174.18696 60.12804) (end 175.886 58.429) (width 1) (layer "B.Cu") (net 5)))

